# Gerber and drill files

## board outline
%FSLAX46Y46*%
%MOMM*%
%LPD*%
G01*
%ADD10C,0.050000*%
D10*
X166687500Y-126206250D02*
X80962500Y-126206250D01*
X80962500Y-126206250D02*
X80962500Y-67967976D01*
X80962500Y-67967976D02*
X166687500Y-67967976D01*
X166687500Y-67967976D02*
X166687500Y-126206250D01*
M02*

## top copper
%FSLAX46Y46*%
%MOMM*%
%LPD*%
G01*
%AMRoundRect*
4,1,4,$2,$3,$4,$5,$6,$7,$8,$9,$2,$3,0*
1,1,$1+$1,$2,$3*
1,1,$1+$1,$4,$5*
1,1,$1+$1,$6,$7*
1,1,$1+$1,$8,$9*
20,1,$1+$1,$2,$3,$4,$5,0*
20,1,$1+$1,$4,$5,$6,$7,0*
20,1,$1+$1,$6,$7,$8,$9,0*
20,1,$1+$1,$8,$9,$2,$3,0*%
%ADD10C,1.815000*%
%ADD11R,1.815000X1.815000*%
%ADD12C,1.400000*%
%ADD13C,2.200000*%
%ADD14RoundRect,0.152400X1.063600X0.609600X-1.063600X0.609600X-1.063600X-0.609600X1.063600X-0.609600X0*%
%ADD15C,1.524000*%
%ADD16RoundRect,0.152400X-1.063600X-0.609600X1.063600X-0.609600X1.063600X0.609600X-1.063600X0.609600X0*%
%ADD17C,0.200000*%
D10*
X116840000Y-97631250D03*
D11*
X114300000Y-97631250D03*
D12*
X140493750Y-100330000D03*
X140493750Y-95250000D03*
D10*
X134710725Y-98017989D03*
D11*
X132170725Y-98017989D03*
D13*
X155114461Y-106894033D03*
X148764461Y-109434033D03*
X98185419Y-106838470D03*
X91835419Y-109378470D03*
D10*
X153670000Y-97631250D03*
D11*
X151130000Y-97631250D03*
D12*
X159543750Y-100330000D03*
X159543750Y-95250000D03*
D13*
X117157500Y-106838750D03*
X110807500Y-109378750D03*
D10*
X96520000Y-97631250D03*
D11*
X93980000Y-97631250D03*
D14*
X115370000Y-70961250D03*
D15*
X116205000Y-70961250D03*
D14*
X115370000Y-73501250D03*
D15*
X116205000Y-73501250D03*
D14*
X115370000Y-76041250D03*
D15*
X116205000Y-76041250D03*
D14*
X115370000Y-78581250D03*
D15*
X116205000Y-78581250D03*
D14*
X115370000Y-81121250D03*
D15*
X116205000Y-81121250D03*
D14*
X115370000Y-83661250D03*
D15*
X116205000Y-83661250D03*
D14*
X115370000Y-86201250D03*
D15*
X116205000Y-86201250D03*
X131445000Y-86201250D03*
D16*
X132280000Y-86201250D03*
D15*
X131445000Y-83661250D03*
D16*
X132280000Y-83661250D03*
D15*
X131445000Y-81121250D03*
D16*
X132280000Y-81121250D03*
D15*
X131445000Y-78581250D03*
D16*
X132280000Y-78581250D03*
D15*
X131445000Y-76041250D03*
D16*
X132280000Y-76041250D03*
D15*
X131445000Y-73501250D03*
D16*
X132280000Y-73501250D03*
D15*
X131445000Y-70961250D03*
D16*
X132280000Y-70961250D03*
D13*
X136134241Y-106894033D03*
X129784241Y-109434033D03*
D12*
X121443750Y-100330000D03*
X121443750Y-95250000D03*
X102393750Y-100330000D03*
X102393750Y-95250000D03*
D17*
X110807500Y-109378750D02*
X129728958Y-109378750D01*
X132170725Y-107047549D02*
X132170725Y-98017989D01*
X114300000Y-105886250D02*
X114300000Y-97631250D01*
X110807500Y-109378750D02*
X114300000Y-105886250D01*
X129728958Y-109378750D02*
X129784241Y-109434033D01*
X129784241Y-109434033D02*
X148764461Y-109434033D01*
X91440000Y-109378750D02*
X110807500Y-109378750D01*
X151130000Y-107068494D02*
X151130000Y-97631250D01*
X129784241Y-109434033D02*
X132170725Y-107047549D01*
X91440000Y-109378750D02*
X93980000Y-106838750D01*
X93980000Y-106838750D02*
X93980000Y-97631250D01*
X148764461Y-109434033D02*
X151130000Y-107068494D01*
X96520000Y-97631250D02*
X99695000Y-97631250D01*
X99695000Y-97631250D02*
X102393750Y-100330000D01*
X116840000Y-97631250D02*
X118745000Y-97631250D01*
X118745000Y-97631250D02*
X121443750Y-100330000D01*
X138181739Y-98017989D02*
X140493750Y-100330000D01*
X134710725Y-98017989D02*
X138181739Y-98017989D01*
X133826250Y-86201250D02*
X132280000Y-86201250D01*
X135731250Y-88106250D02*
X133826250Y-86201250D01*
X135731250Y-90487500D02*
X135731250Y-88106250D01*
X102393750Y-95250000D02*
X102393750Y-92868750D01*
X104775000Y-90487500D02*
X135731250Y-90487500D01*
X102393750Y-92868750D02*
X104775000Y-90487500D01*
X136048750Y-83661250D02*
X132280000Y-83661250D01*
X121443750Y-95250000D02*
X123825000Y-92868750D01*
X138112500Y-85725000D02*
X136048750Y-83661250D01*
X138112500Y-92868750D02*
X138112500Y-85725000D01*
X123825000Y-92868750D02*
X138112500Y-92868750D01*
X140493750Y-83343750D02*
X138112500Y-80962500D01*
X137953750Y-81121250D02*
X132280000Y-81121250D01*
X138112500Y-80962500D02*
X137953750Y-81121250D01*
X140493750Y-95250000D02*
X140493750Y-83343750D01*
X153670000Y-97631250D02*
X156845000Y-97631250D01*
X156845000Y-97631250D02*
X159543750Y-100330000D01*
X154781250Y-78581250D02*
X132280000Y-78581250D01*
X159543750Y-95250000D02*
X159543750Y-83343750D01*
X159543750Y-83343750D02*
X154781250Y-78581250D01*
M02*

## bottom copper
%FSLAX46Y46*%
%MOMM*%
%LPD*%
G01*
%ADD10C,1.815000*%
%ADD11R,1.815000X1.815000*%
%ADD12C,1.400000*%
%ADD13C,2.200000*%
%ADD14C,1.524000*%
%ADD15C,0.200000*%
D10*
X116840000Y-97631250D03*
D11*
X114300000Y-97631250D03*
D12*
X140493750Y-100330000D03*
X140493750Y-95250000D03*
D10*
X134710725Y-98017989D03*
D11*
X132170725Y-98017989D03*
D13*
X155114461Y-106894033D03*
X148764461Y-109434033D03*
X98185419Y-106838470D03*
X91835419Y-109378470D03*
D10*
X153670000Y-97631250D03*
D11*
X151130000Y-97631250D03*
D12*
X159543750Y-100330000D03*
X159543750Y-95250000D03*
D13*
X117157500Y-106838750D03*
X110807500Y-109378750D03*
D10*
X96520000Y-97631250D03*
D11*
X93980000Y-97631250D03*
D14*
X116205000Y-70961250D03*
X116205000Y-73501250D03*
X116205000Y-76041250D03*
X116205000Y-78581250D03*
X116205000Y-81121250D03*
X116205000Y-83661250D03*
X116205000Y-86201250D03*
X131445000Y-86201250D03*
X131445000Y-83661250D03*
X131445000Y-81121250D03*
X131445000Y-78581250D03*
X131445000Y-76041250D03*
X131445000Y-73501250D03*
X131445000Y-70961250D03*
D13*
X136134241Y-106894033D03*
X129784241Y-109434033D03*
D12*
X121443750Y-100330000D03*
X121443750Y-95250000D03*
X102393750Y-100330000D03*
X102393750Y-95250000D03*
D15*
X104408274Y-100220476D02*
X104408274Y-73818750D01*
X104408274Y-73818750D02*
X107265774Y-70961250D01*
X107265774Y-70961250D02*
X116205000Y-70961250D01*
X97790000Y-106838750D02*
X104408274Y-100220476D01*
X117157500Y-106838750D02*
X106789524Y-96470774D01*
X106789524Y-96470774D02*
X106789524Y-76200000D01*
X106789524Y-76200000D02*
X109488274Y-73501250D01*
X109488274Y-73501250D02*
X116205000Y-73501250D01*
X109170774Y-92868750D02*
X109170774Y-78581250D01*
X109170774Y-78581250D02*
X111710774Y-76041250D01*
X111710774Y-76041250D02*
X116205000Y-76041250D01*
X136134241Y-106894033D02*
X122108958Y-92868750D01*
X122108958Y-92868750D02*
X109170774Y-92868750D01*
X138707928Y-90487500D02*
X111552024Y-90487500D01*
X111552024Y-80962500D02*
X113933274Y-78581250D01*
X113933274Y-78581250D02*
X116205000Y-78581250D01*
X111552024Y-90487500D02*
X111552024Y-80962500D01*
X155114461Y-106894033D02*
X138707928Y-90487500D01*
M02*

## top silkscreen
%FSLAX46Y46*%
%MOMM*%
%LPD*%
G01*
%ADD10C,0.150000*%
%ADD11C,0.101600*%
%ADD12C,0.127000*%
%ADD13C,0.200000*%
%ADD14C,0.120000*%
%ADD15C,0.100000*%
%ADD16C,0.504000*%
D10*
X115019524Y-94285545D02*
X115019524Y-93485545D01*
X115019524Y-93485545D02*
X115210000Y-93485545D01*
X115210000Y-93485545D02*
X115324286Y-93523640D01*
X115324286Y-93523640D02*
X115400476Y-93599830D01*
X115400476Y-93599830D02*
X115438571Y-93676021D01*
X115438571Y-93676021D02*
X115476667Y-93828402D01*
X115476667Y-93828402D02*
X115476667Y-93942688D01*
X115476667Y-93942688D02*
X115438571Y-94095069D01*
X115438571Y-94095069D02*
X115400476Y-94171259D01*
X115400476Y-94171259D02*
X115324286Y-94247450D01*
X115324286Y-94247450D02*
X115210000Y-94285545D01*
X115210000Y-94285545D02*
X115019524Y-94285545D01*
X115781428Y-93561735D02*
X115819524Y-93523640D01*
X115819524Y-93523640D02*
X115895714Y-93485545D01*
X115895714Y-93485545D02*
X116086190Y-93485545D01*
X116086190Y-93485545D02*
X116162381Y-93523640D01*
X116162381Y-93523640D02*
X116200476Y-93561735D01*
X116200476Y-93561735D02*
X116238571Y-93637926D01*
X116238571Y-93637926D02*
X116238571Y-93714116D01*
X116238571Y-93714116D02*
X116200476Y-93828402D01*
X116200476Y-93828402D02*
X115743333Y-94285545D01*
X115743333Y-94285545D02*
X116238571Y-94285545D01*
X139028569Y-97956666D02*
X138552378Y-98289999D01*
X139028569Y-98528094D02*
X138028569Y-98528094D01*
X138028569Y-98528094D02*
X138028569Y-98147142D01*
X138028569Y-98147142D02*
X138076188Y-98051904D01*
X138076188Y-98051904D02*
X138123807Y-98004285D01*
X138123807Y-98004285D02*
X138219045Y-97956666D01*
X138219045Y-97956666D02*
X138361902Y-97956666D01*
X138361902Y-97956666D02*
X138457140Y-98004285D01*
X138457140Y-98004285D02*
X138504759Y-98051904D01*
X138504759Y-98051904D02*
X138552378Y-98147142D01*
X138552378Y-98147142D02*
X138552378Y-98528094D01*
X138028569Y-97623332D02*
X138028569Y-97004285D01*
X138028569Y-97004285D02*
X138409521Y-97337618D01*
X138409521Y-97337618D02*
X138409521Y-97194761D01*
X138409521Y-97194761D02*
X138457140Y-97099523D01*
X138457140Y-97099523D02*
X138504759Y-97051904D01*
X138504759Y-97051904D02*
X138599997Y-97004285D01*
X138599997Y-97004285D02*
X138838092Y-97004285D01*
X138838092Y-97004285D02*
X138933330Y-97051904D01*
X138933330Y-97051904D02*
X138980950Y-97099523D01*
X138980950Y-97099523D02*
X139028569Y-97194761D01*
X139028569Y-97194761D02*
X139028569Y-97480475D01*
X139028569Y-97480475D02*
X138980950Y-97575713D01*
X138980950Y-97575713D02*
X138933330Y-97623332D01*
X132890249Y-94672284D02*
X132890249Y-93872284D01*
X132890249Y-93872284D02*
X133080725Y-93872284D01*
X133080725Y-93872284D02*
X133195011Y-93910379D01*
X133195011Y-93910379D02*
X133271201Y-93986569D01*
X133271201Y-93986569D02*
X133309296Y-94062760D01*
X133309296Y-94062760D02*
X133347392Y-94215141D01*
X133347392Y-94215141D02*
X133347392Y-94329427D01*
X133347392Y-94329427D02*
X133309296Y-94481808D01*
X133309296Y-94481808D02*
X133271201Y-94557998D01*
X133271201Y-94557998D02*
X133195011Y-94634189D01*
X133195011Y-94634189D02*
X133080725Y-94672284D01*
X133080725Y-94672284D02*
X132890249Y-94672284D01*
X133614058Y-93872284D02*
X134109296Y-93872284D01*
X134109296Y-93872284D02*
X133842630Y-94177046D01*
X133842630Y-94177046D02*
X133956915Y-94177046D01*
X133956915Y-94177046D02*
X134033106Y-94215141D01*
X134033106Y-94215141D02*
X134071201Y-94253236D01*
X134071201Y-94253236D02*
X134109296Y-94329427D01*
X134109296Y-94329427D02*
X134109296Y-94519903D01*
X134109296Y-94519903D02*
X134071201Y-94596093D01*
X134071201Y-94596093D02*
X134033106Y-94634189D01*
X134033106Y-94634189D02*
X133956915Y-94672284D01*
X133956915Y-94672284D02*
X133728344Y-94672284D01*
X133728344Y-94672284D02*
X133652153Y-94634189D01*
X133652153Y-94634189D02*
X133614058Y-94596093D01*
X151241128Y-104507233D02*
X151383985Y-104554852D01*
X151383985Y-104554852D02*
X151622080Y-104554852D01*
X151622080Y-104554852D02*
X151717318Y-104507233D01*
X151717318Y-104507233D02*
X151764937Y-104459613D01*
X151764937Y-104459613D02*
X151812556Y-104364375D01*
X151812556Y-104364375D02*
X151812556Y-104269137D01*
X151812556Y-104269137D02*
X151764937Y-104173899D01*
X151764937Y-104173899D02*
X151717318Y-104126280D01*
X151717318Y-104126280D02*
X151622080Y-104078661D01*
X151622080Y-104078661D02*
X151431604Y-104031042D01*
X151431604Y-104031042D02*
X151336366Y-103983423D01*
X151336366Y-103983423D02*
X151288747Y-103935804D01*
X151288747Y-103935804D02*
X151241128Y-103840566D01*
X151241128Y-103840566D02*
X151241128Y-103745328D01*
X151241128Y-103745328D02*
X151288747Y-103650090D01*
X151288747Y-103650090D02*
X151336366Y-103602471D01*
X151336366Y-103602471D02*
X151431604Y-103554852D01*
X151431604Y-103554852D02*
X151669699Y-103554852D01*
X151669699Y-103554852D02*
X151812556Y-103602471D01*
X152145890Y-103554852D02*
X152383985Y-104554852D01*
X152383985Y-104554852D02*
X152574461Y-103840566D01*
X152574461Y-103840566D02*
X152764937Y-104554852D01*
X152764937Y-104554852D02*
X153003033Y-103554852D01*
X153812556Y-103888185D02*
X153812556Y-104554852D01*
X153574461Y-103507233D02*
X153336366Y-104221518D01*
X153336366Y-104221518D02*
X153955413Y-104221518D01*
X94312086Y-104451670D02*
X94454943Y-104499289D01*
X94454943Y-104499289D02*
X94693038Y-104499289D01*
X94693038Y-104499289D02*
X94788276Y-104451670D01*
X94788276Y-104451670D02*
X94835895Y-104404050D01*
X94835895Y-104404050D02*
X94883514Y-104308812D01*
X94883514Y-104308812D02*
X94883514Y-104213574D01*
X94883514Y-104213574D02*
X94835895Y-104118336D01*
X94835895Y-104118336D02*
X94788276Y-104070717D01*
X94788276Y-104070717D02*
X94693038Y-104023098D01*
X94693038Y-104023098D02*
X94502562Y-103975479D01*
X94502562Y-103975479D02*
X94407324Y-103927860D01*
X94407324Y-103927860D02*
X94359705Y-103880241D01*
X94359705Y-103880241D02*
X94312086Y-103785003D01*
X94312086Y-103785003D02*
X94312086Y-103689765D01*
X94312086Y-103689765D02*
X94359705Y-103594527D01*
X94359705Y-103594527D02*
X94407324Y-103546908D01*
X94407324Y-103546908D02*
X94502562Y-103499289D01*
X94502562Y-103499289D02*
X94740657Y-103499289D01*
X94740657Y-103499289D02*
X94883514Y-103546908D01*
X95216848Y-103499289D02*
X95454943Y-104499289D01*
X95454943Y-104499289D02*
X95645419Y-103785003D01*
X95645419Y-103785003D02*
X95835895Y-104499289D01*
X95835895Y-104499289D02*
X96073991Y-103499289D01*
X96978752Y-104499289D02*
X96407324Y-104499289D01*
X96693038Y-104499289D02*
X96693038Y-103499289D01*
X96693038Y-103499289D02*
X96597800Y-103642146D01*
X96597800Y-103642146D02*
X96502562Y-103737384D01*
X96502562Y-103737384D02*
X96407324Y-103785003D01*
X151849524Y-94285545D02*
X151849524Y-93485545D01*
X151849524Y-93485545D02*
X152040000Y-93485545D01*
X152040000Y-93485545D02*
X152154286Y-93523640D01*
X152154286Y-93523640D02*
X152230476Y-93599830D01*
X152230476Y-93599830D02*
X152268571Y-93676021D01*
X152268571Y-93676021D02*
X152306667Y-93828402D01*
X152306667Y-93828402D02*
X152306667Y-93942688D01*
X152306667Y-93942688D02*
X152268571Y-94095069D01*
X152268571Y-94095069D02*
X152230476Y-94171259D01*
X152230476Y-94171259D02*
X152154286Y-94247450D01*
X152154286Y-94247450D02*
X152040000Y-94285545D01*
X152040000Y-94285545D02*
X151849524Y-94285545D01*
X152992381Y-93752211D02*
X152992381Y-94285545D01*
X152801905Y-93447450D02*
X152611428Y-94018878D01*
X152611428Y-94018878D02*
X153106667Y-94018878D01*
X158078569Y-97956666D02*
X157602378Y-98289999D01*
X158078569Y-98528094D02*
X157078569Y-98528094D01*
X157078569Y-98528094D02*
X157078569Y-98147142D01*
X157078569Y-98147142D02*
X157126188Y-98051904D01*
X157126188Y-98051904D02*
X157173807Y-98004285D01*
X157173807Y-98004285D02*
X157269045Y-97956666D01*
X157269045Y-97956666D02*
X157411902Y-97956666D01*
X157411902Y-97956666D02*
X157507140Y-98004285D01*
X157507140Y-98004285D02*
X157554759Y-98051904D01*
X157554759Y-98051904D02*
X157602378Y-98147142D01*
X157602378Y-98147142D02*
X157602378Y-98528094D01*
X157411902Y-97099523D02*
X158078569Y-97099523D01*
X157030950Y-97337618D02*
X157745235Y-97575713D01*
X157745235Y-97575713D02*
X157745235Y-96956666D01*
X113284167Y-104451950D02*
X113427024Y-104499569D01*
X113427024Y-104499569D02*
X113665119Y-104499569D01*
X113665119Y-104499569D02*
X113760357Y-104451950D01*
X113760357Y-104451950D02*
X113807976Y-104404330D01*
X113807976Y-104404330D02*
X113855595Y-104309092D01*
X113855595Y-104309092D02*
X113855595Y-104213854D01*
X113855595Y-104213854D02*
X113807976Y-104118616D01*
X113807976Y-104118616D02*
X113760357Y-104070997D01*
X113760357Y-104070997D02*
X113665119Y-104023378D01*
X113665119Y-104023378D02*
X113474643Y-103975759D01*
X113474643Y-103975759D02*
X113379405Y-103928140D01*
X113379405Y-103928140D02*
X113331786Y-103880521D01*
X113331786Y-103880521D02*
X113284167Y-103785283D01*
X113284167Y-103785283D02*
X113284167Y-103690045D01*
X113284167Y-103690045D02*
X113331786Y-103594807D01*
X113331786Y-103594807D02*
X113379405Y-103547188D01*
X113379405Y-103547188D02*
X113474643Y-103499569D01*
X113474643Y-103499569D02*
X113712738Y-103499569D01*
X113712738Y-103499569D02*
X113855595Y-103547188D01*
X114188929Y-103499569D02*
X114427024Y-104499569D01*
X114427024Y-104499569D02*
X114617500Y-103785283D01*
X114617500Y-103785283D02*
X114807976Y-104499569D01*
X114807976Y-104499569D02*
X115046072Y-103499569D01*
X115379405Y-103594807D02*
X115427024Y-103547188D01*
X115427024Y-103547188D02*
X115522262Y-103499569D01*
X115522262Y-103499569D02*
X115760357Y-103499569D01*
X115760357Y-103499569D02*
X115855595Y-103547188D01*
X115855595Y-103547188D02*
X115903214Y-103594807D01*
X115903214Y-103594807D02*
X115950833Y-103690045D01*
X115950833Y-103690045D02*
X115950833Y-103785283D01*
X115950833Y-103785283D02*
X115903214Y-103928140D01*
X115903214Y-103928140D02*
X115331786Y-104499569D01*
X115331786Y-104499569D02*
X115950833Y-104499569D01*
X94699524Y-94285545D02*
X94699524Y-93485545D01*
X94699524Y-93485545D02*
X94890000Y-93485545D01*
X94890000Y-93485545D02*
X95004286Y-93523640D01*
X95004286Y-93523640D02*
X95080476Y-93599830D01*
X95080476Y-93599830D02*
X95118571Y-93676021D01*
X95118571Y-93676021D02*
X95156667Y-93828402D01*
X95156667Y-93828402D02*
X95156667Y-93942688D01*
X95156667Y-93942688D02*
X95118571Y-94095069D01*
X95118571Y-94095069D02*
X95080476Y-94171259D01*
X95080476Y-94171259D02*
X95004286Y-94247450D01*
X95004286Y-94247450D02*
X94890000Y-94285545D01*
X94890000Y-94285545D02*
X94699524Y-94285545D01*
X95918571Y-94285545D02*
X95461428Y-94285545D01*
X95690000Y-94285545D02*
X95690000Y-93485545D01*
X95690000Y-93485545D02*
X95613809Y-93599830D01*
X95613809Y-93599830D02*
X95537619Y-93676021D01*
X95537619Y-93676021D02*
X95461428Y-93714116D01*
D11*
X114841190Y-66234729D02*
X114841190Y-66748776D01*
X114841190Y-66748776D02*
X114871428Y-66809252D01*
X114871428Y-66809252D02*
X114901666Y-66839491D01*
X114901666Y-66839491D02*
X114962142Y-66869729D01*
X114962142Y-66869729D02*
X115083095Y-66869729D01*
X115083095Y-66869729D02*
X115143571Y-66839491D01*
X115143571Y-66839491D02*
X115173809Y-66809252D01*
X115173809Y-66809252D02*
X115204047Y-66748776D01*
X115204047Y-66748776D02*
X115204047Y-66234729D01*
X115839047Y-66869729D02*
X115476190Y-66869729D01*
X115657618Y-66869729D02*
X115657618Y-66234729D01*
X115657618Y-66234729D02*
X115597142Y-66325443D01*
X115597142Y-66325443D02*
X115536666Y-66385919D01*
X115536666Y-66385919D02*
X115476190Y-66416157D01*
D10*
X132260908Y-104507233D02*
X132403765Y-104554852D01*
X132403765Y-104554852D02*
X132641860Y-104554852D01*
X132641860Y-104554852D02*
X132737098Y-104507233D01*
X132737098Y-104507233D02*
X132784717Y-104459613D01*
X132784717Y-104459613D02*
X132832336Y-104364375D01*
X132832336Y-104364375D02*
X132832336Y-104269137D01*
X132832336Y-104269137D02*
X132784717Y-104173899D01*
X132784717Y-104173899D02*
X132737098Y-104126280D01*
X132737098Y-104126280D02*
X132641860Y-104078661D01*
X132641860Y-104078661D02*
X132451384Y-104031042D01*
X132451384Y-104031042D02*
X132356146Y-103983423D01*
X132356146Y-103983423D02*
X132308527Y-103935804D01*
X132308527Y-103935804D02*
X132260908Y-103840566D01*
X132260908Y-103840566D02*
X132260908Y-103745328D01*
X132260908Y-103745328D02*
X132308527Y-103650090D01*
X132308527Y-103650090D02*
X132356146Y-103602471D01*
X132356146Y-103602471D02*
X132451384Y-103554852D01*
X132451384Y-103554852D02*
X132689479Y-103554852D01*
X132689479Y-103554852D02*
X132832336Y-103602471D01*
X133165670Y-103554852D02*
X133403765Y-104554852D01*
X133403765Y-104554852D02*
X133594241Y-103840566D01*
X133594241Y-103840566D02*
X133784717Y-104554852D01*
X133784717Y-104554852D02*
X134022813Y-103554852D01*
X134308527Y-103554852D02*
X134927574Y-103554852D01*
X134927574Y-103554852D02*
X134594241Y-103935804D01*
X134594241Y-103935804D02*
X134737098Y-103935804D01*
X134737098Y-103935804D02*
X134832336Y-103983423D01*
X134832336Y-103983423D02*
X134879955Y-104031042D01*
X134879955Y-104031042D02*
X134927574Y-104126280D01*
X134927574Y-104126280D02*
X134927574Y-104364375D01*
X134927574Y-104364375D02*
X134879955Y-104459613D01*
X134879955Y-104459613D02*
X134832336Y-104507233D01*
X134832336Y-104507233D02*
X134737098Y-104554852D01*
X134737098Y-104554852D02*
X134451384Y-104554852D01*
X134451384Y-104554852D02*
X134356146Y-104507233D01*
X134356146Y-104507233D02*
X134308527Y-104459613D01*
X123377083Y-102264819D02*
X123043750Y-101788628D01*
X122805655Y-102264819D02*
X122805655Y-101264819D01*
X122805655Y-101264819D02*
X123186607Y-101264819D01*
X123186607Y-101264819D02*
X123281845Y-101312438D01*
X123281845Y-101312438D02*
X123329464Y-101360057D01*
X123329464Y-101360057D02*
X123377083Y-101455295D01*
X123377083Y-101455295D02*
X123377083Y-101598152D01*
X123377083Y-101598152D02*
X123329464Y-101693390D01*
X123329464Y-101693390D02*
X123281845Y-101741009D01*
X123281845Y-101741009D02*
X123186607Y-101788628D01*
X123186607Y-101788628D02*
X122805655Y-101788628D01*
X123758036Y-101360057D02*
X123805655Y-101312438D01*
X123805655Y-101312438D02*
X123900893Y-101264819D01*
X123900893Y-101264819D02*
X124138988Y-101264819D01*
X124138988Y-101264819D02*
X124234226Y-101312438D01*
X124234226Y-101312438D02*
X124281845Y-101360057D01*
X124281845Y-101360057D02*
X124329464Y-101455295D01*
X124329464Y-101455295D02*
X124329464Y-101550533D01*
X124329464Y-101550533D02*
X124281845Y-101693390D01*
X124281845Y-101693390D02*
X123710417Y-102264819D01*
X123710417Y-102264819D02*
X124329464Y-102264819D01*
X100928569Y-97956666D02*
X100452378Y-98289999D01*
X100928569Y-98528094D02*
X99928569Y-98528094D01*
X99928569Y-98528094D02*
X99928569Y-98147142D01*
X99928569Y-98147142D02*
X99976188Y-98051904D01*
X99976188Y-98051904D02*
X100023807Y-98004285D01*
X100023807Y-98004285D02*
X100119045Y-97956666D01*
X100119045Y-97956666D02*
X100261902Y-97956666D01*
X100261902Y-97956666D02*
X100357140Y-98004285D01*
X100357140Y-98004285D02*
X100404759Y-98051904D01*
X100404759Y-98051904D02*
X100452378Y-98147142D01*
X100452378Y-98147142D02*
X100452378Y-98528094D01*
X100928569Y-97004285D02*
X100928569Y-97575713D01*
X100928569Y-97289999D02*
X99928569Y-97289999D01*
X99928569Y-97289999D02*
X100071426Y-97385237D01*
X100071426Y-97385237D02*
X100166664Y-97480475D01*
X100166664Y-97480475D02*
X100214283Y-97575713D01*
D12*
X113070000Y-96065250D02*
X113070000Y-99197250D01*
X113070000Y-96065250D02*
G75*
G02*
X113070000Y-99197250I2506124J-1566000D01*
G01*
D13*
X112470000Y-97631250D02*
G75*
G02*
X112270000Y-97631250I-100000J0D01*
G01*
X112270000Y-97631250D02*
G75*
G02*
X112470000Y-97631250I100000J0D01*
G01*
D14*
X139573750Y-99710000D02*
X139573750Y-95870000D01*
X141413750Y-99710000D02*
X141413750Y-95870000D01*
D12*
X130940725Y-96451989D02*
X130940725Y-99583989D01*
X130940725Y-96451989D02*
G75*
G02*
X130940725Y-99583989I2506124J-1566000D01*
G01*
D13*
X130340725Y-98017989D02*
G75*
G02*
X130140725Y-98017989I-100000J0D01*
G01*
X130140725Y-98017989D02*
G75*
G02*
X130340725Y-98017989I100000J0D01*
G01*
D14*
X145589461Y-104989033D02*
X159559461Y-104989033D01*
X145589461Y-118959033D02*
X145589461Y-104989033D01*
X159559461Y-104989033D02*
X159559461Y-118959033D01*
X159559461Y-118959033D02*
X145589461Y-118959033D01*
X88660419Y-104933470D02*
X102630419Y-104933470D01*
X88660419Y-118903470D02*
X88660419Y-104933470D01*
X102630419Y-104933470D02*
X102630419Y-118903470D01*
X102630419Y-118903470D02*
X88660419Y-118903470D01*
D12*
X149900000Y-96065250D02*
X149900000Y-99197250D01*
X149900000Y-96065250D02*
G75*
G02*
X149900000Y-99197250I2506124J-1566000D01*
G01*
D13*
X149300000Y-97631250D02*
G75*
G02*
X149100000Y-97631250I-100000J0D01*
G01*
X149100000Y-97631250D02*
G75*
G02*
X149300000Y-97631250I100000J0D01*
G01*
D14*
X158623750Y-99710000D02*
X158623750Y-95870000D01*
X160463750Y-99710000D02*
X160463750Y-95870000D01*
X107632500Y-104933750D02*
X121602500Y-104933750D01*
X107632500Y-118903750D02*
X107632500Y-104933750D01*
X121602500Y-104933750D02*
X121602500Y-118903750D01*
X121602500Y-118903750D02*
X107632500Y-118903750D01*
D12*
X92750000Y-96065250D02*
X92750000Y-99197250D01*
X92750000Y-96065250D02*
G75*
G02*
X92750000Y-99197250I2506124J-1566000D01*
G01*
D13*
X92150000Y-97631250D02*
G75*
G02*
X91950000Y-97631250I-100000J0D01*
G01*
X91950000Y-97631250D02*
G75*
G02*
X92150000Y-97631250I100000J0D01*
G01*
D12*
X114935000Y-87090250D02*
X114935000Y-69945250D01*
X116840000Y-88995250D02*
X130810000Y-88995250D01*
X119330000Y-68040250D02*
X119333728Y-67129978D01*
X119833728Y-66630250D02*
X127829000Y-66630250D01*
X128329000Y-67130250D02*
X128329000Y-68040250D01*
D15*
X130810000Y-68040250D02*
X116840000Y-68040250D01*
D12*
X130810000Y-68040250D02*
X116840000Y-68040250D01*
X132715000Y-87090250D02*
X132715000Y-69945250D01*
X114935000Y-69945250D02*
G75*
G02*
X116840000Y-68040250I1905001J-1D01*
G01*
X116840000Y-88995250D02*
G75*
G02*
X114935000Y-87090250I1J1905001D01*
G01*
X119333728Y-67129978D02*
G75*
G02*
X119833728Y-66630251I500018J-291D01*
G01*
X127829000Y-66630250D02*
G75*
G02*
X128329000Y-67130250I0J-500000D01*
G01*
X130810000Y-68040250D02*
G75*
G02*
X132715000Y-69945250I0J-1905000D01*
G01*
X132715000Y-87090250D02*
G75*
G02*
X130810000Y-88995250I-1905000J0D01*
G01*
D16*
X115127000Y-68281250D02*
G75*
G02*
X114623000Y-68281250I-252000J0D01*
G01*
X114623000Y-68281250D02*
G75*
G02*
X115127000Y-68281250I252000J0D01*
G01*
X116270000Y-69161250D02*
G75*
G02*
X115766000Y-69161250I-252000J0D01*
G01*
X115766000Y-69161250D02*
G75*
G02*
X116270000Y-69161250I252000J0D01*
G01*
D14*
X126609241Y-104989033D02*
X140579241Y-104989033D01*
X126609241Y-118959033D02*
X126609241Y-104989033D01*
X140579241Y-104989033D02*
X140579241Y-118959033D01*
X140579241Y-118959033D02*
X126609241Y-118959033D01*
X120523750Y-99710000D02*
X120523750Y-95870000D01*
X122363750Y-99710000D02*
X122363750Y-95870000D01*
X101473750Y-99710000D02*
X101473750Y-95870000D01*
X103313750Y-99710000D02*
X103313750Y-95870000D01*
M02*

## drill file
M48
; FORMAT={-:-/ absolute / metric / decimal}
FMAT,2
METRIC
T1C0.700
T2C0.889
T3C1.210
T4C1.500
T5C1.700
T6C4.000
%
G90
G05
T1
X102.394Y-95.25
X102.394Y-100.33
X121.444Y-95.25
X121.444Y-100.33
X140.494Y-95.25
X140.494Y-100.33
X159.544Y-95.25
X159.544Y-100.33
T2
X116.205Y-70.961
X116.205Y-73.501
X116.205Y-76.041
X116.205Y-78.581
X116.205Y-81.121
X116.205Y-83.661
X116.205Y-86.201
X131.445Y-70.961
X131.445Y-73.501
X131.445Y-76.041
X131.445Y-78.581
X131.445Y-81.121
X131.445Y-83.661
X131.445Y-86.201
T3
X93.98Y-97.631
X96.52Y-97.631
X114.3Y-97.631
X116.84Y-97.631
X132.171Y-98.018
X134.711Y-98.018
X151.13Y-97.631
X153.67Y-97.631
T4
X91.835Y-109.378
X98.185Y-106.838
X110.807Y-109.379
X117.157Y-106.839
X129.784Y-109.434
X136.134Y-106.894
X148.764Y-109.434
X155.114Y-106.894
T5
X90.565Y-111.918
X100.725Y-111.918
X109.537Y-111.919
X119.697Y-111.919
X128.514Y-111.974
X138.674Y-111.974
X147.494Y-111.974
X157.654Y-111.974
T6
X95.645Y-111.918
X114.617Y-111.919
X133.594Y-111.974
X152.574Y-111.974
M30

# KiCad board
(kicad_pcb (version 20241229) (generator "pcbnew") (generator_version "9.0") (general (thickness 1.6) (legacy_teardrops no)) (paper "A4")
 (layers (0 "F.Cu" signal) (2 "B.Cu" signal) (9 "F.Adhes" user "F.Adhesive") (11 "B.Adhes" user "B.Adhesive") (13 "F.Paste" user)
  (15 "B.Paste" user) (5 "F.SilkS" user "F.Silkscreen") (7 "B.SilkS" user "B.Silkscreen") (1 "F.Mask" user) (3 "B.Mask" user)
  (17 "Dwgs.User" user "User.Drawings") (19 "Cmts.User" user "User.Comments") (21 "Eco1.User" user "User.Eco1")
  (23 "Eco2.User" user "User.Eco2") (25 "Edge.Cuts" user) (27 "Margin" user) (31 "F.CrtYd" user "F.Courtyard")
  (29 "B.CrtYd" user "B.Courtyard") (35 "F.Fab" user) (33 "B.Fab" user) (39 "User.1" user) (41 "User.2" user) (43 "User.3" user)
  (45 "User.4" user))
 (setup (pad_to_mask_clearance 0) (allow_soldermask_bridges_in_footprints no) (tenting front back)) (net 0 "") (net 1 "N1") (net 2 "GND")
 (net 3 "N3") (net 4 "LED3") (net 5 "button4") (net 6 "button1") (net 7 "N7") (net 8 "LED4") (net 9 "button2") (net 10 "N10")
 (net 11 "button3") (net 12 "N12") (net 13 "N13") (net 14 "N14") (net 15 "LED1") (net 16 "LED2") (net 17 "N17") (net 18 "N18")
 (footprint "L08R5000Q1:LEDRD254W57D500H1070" (layer "F.Cu") (at 115.57 97.63125)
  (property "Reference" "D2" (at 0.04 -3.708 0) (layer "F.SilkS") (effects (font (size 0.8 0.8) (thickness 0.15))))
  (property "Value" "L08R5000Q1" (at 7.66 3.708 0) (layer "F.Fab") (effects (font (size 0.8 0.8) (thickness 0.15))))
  (fp_line (start -2.5 -1.566) (end -2.5 1.566) (stroke (width 0.127) (type solid)) (layer "F.SilkS"))
  (fp_arc (start -2.5 -1.566) (mid 2.961291 0) (end -2.5 1.566) (stroke (width 0.127) (type solid)) (layer "F.SilkS"))
  (fp_circle (center -3.2 0) (end -3.1 0) (stroke (width 0.2) (type solid)) (fill no) (layer "F.SilkS"))
  (pad "A" thru_hole circle (at 1.27 0) (size 1.815 1.815) (drill 1.21) (layers "*.Cu" "*.Mask") (remove_unused_layers no) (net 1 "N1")
   (solder_mask_margin 0.102))
  (pad "C" thru_hole rect (at -1.27 0) (size 1.815 1.815) (drill 1.21) (layers "*.Cu" "*.Mask") (remove_unused_layers no) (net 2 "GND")
   (solder_mask_margin 0.102)))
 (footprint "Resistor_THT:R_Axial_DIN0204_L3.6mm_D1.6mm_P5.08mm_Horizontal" (layer "F.Cu") (at 140.49375 100.33 90)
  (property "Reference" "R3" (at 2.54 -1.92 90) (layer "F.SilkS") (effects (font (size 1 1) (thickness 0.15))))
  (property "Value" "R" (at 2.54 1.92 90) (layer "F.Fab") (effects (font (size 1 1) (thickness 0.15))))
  (fp_line (start 0.62 -0.92) (end 4.46 -0.92) (stroke (width 0.12) (type solid)) (layer "F.SilkS"))
  (fp_line (start 0.62 0.92) (end 4.46 0.92) (stroke (width 0.12) (type solid)) (layer "F.SilkS"))
  (pad "1" thru_hole circle (at 0 0 90) (size 1.4 1.4) (drill 0.7) (layers "*.Cu" "*.Mask") (remove_unused_layers no) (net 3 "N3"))
  (pad "2" thru_hole circle (at 5.08 0 90) (size 1.4 1.4) (drill 0.7) (layers "*.Cu" "*.Mask") (remove_unused_layers no) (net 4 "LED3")))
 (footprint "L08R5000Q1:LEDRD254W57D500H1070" (layer "F.Cu") (at 133.440725 98.017989)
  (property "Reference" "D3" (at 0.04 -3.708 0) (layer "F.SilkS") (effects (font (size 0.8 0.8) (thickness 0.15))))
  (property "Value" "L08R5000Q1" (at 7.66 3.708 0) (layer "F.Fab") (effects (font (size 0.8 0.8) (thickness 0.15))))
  (fp_line (start -2.5 -1.566) (end -2.5 1.566) (stroke (width 0.127) (type solid)) (layer "F.SilkS"))
  (fp_arc (start -2.5 -1.566) (mid 2.961291 0) (end -2.5 1.566) (stroke (width 0.127) (type solid)) (layer "F.SilkS"))
  (fp_circle (center -3.2 0) (end -3.1 0) (stroke (width 0.2) (type solid)) (fill no) (layer "F.SilkS"))
  (pad "A" thru_hole circle (at 1.27 0) (size 1.815 1.815) (drill 1.21) (layers "*.Cu" "*.Mask") (remove_unused_layers no) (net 3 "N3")
   (solder_mask_margin 0.102))
  (pad "C" thru_hole rect (at -1.27 0) (size 1.815 1.815) (drill 1.21) (layers "*.Cu" "*.Mask") (remove_unused_layers no) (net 2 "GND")
   (solder_mask_margin 0.102)))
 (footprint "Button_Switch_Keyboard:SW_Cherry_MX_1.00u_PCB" (layer "F.Cu") (at 155.114461 106.894033)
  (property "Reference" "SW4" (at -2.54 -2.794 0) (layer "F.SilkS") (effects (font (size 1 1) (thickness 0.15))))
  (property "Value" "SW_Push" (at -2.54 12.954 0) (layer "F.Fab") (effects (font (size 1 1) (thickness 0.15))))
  (fp_line (start -9.525 -1.905) (end 4.445 -1.905) (stroke (width 0.12) (type solid)) (layer "F.SilkS"))
  (fp_line (start -9.525 12.065) (end -9.525 -1.905) (stroke (width 0.12) (type solid)) (layer "F.SilkS"))
  (fp_line (start 4.445 -1.905) (end 4.445 12.065) (stroke (width 0.12) (type solid)) (layer "F.SilkS"))
  (fp_line (start 4.445 12.065) (end -9.525 12.065) (stroke (width 0.12) (type solid)) (layer "F.SilkS"))
  (pad "" np_thru_hole circle (at -7.62 5.08) (size 1.7 1.7) (drill 1.7) (layers "*.Cu" "*.Mask"))
  (pad "" np_thru_hole circle (at -2.54 5.08) (size 4 4) (drill 4) (layers "*.Cu" "*.Mask"))
  (pad "" np_thru_hole circle (at 2.54 5.08) (size 1.7 1.7) (drill 1.7) (layers "*.Cu" "*.Mask"))
  (pad "1" thru_hole circle (at 0 0) (size 2.2 2.2) (drill 1.5) (layers "*.Cu" "*.Mask") (remove_unused_layers no) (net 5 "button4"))
  (pad "2" thru_hole circle (at -6.35 2.54) (size 2.2 2.2) (drill 1.5) (layers "*.Cu" "*.Mask") (remove_unused_layers no) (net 2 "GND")))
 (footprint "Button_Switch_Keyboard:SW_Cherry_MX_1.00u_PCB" (layer "F.Cu") (at 98.185419 106.83847)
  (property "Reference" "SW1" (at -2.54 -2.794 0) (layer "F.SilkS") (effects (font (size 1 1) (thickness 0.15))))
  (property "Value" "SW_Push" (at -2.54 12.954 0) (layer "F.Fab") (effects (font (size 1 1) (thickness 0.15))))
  (fp_line (start -9.525 -1.905) (end 4.445 -1.905) (stroke (width 0.12) (type solid)) (layer "F.SilkS"))
  (fp_line (start -9.525 12.065) (end -9.525 -1.905) (stroke (width 0.12) (type solid)) (layer "F.SilkS"))
  (fp_line (start 4.445 -1.905) (end 4.445 12.065) (stroke (width 0.12) (type solid)) (layer "F.SilkS"))
  (fp_line (start 4.445 12.065) (end -9.525 12.065) (stroke (width 0.12) (type solid)) (layer "F.SilkS"))
  (pad "" np_thru_hole circle (at -7.62 5.08) (size 1.7 1.7) (drill 1.7) (layers "*.Cu" "*.Mask"))
  (pad "" np_thru_hole circle (at -2.54 5.08) (size 4 4) (drill 4) (layers "*.Cu" "*.Mask"))
  (pad "" np_thru_hole circle (at 2.54 5.08) (size 1.7 1.7) (drill 1.7) (layers "*.Cu" "*.Mask"))
  (pad "1" thru_hole circle (at 0 0) (size 2.2 2.2) (drill 1.5) (layers "*.Cu" "*.Mask") (remove_unused_layers no) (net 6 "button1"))
  (pad "2" thru_hole circle (at -6.35 2.54) (size 2.2 2.2) (drill 1.5) (layers "*.Cu" "*.Mask") (remove_unused_layers no) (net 2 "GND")))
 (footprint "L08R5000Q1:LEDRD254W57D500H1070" (layer "F.Cu") (at 152.4 97.63125)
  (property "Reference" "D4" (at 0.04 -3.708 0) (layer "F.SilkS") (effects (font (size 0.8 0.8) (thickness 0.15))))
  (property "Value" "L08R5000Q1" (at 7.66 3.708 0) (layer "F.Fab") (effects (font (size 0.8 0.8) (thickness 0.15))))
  (fp_line (start -2.5 -1.566) (end -2.5 1.566) (stroke (width 0.127) (type solid)) (layer "F.SilkS"))
  (fp_arc (start -2.5 -1.566) (mid 2.961291 0) (end -2.5 1.566) (stroke (width 0.127) (type solid)) (layer "F.SilkS"))
  (fp_circle (center -3.2 0) (end -3.1 0) (stroke (width 0.2) (type solid)) (fill no) (layer "F.SilkS"))
  (pad "A" thru_hole circle (at 1.27 0) (size 1.815 1.815) (drill 1.21) (layers "*.Cu" "*.Mask") (remove_unused_layers no) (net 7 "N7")
   (solder_mask_margin 0.102))
  (pad "C" thru_hole rect (at -1.27 0) (size 1.815 1.815) (drill 1.21) (layers "*.Cu" "*.Mask") (remove_unused_layers no) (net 2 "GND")
   (solder_mask_margin 0.102)))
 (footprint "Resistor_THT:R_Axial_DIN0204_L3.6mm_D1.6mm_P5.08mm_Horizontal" (layer "F.Cu") (at 159.54375 100.33 90)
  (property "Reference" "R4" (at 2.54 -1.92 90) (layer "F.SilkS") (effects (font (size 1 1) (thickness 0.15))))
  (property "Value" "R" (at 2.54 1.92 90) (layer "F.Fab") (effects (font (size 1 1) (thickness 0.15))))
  (fp_line (start 0.62 -0.92) (end 4.46 -0.92) (stroke (width 0.12) (type solid)) (layer "F.SilkS"))
  (fp_line (start 0.62 0.92) (end 4.46 0.92) (stroke (width 0.12) (type solid)) (layer "F.SilkS"))
  (pad "1" thru_hole circle (at 0 0 90) (size 1.4 1.4) (drill 0.7) (layers "*.Cu" "*.Mask") (remove_unused_layers no) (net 7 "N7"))
  (pad "2" thru_hole circle (at 5.08 0 90) (size 1.4 1.4) (drill 0.7) (layers "*.Cu" "*.Mask") (remove_unused_layers no) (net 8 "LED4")))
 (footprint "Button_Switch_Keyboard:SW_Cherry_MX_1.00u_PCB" (layer "F.Cu") (at 117.1575 106.83875)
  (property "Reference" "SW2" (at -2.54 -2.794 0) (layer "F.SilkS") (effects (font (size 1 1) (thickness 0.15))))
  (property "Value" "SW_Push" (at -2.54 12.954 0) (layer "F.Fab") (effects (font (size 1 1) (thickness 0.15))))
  (fp_line (start -9.525 -1.905) (end 4.445 -1.905) (stroke (width 0.12) (type solid)) (layer "F.SilkS"))
  (fp_line (start -9.525 12.065) (end -9.525 -1.905) (stroke (width 0.12) (type solid)) (layer "F.SilkS"))
  (fp_line (start 4.445 -1.905) (end 4.445 12.065) (stroke (width 0.12) (type solid)) (layer "F.SilkS"))
  (fp_line (start 4.445 12.065) (end -9.525 12.065) (stroke (width 0.12) (type solid)) (layer "F.SilkS"))
  (pad "" np_thru_hole circle (at -7.62 5.08) (size 1.7 1.7) (drill 1.7) (layers "*.Cu" "*.Mask"))
  (pad "" np_thru_hole circle (at -2.54 5.08) (size 4 4) (drill 4) (layers "*.Cu" "*.Mask"))
  (pad "" np_thru_hole circle (at 2.54 5.08) (size 1.7 1.7) (drill 1.7) (layers "*.Cu" "*.Mask"))
  (pad "1" thru_hole circle (at 0 0) (size 2.2 2.2) (drill 1.5) (layers "*.Cu" "*.Mask") (remove_unused_layers no) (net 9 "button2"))
  (pad "2" thru_hole circle (at -6.35 2.54) (size 2.2 2.2) (drill 1.5) (layers "*.Cu" "*.Mask") (remove_unused_layers no) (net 2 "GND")))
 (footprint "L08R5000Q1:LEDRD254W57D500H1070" (layer "F.Cu") (at 95.25 97.63125)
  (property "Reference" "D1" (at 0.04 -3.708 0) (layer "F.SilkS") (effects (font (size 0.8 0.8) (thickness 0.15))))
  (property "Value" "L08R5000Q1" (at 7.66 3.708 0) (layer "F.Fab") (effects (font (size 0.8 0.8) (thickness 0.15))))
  (fp_line (start -2.5 -1.566) (end -2.5 1.566) (stroke (width 0.127) (type solid)) (layer "F.SilkS"))
  (fp_arc (start -2.5 -1.566) (mid 2.961291 0) (end -2.5 1.566) (stroke (width 0.127) (type solid)) (layer "F.SilkS"))
  (fp_circle (center -3.2 0) (end -3.1 0) (stroke (width 0.2) (type solid)) (fill no) (layer "F.SilkS"))
  (pad "A" thru_hole circle (at 1.27 0) (size 1.815 1.815) (drill 1.21) (layers "*.Cu" "*.Mask") (remove_unused_layers no) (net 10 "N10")
   (solder_mask_margin 0.102))
  (pad "C" thru_hole rect (at -1.27 0) (size 1.815 1.815) (drill 1.21) (layers "*.Cu" "*.Mask") (remove_unused_layers no) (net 2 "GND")
   (solder_mask_margin 0.102)))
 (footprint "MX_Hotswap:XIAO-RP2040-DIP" (layer "F.Cu") (at 123.825 78.58125)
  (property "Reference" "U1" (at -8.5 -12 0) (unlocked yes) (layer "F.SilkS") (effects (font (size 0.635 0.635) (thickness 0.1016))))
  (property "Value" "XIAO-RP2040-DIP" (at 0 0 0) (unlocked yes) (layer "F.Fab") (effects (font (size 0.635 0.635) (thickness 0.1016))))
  (fp_line (start -8.89 8.509) (end -8.89 -8.636) (stroke (width 0.127) (type solid)) (layer "F.SilkS"))
  (fp_line (start -6.985 10.414) (end 6.985 10.414) (stroke (width 0.127) (type solid)) (layer "F.SilkS"))
  (fp_line (start -4.495 -10.541) (end -4.491272 -11.451272) (stroke (width 0.127) (type solid)) (layer "F.SilkS"))
  (fp_line (start -3.991272 -11.951) (end 4.004 -11.951) (stroke (width 0.127) (type solid)) (layer "F.SilkS"))
  (fp_line (start 4.504 -11.451) (end 4.504 -10.541) (stroke (width 0.127) (type solid)) (layer "F.SilkS"))
  (fp_line (start 6.985 -10.541) (end -6.985 -10.541) (stroke (width 0.1) (type solid)) (layer "F.SilkS"))
  (fp_line (start 6.985 -10.541) (end -6.985 -10.541) (stroke (width 0.127) (type solid)) (layer "F.SilkS"))
  (fp_line (start 8.89 8.509) (end 8.89 -8.636) (stroke (width 0.127) (type solid)) (layer "F.SilkS"))
  (fp_arc (start -8.89 -8.636) (mid -8.332038 -9.983038) (end -6.985 -10.541) (stroke (width 0.127) (type solid)) (layer "F.SilkS"))
  (fp_arc (start -6.985 10.414) (mid -8.332038 9.856038) (end -8.89 8.509) (stroke (width 0.127) (type solid)) (layer "F.SilkS"))
  (fp_arc (start -4.491272 -11.451272) (mid -4.344728 -11.80464) (end -3.991272 -11.951) (stroke (width 0.127) (type default))
   (layer "F.SilkS"))
  (fp_arc (start 4.004 -11.951) (mid 4.357553 -11.804553) (end 4.504 -11.451) (stroke (width 0.127) (type default)) (layer "F.SilkS"))
  (fp_arc (start 6.985 -10.541) (mid 8.332038 -9.983038) (end 8.89 -8.636) (stroke (width 0.127) (type solid)) (layer "F.SilkS"))
  (fp_arc (start 8.89 8.509) (mid 8.332038 9.856038) (end 6.985 10.414) (stroke (width 0.127) (type solid)) (layer "F.SilkS"))
  (fp_circle (center -8.95 -10.3) (end -8.95 -10.554) (stroke (width 0.5) (type solid)) (fill yes) (layer "F.SilkS"))
  (fp_circle (center -7.807 -9.42) (end -7.807 -9.674) (stroke (width 0.5) (type solid)) (fill yes) (layer "F.SilkS"))
  (pad "1" smd roundrect (at -8.455 -7.62 180) (size 2.432 1.524) (layers "F.Cu" "F.Mask") (roundrect_rratio 0.1) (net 6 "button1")
   (thermal_bridge_angle 45))
  (pad "1" thru_hole circle (at -7.62 -7.62 180) (size 1.524 1.524) (drill 0.889) (layers "*.Cu" "*.Mask") (remove_unused_layers no)
   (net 6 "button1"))
  (pad "2" smd roundrect (at -8.455 -5.08 180) (size 2.432 1.524) (layers "F.Cu" "F.Mask") (roundrect_rratio 0.1) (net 9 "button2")
   (thermal_bridge_angle 45))
  (pad "2" thru_hole circle (at -7.62 -5.08 180) (size 1.524 1.524) (drill 0.889) (layers "*.Cu" "*.Mask") (remove_unused_layers no)
   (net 9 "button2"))
  (pad "3" smd roundrect (at -8.455 -2.54 180) (size 2.432 1.524) (layers "F.Cu" "F.Mask") (roundrect_rratio 0.1) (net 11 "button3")
   (thermal_bridge_angle 45))
  (pad "3" thru_hole circle (at -7.62 -2.54 180) (size 1.524 1.524) (drill 0.889) (layers "*.Cu" "*.Mask") (remove_unused_layers no)
   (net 11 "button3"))
  (pad "4" smd roundrect (at -8.455 0 180) (size 2.432 1.524) (layers "F.Cu" "F.Mask") (roundrect_rratio 0.1) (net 5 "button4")
   (thermal_bridge_angle 45))
  (pad "4" thru_hole circle (at -7.62 0 180) (size 1.524 1.524) (drill 0.889) (layers "*.Cu" "*.Mask") (remove_unused_layers no)
   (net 5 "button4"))
  (pad "5" smd roundrect (at -8.455 2.54 180) (size 2.432 1.524) (layers "F.Cu" "F.Mask") (roundrect_rratio 0.1) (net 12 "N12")
   (thermal_bridge_angle 45))
  (pad "5" thru_hole circle (at -7.62 2.54 180) (size 1.524 1.524) (drill 0.889) (layers "*.Cu" "*.Mask") (remove_unused_layers no)
   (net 12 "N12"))
  (pad "6" smd roundrect (at -8.455 5.08 180) (size 2.432 1.524) (layers "F.Cu" "F.Mask") (roundrect_rratio 0.1) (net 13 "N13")
   (thermal_bridge_angle 45))
  (pad "6" thru_hole circle (at -7.62 5.08 180) (size 1.524 1.524) (drill 0.889) (layers "*.Cu" "*.Mask") (remove_unused_layers no)
   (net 13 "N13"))
  (pad "7" smd roundrect (at -8.455 7.62 180) (size 2.432 1.524) (layers "F.Cu" "F.Mask") (roundrect_rratio 0.1) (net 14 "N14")
   (thermal_bridge_angle 45))
  (pad "7" thru_hole circle (at -7.62 7.62 180) (size 1.524 1.524) (drill 0.889) (layers "*.Cu" "*.Mask") (remove_unused_layers no)
   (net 14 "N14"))
  (pad "8" thru_hole circle (at 7.62 7.62) (size 1.524 1.524) (drill 0.889) (layers "*.Cu" "*.Mask") (remove_unused_layers no)
   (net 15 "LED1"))
  (pad "8" smd roundrect (at 8.455 7.62) (size 2.432 1.524) (layers "F.Cu" "F.Mask") (roundrect_rratio 0.1) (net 15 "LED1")
   (thermal_bridge_angle 45))
  (pad "9" thru_hole circle (at 7.62 5.08) (size 1.524 1.524) (drill 0.889) (layers "*.Cu" "*.Mask") (remove_unused_layers no)
   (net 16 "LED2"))
  (pad "9" smd roundrect (at 8.455 5.08) (size 2.432 1.524) (layers "F.Cu" "F.Mask") (roundrect_rratio 0.1) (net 16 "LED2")
   (thermal_bridge_angle 45))
  (pad "10" thru_hole circle (at 7.62 2.54) (size 1.524 1.524) (drill 0.889) (layers "*.Cu" "*.Mask") (remove_unused_layers no)
   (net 4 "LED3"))
  (pad "10" smd roundrect (at 8.455 2.54) (size 2.432 1.524) (layers "F.Cu" "F.Mask") (roundrect_rratio 0.1) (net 4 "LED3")
   (thermal_bridge_angle 45))
  (pad "11" thru_hole circle (at 7.62 0) (size 1.524 1.524) (drill 0.889) (layers "*.Cu" "*.Mask") (remove_unused_layers no) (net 8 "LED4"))
  (pad "11" smd roundrect (at 8.455 0) (size 2.432 1.524) (layers "F.Cu" "F.Mask") (roundrect_rratio 0.1) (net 8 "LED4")
   (thermal_bridge_angle 45))
  (pad "12" thru_hole circle (at 7.62 -2.54) (size 1.524 1.524) (drill 0.889) (layers "*.Cu" "*.Mask") (remove_unused_layers no)
   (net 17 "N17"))
  (pad "12" smd roundrect (at 8.455 -2.54) (size 2.432 1.524) (layers "F.Cu" "F.Mask") (roundrect_rratio 0.1) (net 17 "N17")
   (thermal_bridge_angle 45))
  (pad "13" thru_hole circle (at 7.62 -5.08) (size 1.524 1.524) (drill 0.889) (layers "*.Cu" "*.Mask") (remove_unused_layers no)
   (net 2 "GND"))
  (pad "13" smd roundrect (at 8.455 -5.08) (size 2.432 1.524) (layers "F.Cu" "F.Mask") (roundrect_rratio 0.1) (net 2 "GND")
   (thermal_bridge_angle 45))
  (pad "14" thru_hole circle (at 7.62 -7.62) (size 1.524 1.524) (drill 0.889) (layers "*.Cu" "*.Mask") (remove_unused_layers no)
   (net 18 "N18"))
  (pad "14" smd roundrect (at 8.455 -7.62) (size 2.432 1.524) (layers "F.Cu" "F.Mask") (roundrect_rratio 0.1) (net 18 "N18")
   (thermal_bridge_angle 45)))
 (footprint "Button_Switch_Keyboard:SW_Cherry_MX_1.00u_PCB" (layer "F.Cu") (at 136.134241 106.894033)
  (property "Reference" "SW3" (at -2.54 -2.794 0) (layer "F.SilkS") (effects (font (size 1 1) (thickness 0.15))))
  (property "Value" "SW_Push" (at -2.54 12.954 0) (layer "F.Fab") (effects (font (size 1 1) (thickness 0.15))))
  (fp_line (start -9.525 -1.905) (end 4.445 -1.905) (stroke (width 0.12) (type solid)) (layer "F.SilkS"))
  (fp_line (start -9.525 12.065) (end -9.525 -1.905) (stroke (width 0.12) (type solid)) (layer "F.SilkS"))
  (fp_line (start 4.445 -1.905) (end 4.445 12.065) (stroke (width 0.12) (type solid)) (layer "F.SilkS"))
  (fp_line (start 4.445 12.065) (end -9.525 12.065) (stroke (width 0.12) (type solid)) (layer "F.SilkS"))
  (pad "" np_thru_hole circle (at -7.62 5.08) (size 1.7 1.7) (drill 1.7) (layers "*.Cu" "*.Mask"))
  (pad "" np_thru_hole circle (at -2.54 5.08) (size 4 4) (drill 4) (layers "*.Cu" "*.Mask"))
  (pad "" np_thru_hole circle (at 2.54 5.08) (size 1.7 1.7) (drill 1.7) (layers "*.Cu" "*.Mask"))
  (pad "1" thru_hole circle (at 0 0) (size 2.2 2.2) (drill 1.5) (layers "*.Cu" "*.Mask") (remove_unused_layers no) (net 11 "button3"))
  (pad "2" thru_hole circle (at -6.35 2.54) (size 2.2 2.2) (drill 1.5) (layers "*.Cu" "*.Mask") (remove_unused_layers no) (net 2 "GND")))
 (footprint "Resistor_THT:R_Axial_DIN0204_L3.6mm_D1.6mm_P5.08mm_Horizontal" (layer "F.Cu") (at 121.44375 100.33 90)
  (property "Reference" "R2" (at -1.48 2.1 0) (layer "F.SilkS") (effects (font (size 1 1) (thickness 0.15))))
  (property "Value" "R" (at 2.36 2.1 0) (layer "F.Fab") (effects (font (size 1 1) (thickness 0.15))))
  (fp_line (start 0.62 -0.92) (end 4.46 -0.92) (stroke (width 0.12) (type solid)) (layer "F.SilkS"))
  (fp_line (start 0.62 0.92) (end 4.46 0.92) (stroke (width 0.12) (type solid)) (layer "F.SilkS"))
  (pad "1" thru_hole circle (at 0 0 90) (size 1.4 1.4) (drill 0.7) (layers "*.Cu" "*.Mask") (remove_unused_layers no) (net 1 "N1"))
  (pad "2" thru_hole circle (at 5.08 0 90) (size 1.4 1.4) (drill 0.7) (layers "*.Cu" "*.Mask") (remove_unused_layers no) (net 16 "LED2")))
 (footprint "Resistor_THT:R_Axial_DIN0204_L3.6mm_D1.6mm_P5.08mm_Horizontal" (layer "F.Cu") (at 102.39375 100.33 90)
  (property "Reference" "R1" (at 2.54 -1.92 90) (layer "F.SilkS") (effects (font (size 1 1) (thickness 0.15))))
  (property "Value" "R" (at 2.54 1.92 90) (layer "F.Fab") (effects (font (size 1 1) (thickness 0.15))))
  (fp_line (start 0.62 -0.92) (end 4.46 -0.92) (stroke (width 0.12) (type solid)) (layer "F.SilkS"))
  (fp_line (start 0.62 0.92) (end 4.46 0.92) (stroke (width 0.12) (type solid)) (layer "F.SilkS"))
  (pad "1" thru_hole circle (at 0 0 90) (size 1.4 1.4) (drill 0.7) (layers "*.Cu" "*.Mask") (remove_unused_layers no) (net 10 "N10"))
  (pad "2" thru_hole circle (at 5.08 0 90) (size 1.4 1.4) (drill 0.7) (layers "*.Cu" "*.Mask") (remove_unused_layers no) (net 15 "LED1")))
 (gr_line (start 166.6875 126.20625) (end 80.9625 126.20625) (stroke (width 0.05) (type default)) (layer "Edge.Cuts"))
 (gr_line (start 80.9625 126.20625) (end 80.9625 67.967976) (stroke (width 0.05) (type default)) (layer "Edge.Cuts"))
 (gr_line (start 80.9625 67.967976) (end 166.6875 67.967976) (stroke (width 0.05) (type default)) (layer "Edge.Cuts"))
 (gr_line (start 166.6875 67.967976) (end 166.6875 126.20625) (stroke (width 0.05) (type default)) (layer "Edge.Cuts"))
 (segment (start 110.8075 109.37875) (end 129.728958 109.37875) (width 0.2) (layer "F.Cu") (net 2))
 (segment (start 132.170725 107.047549) (end 132.170725 98.017989) (width 0.2) (layer "F.Cu") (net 2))
 (segment (start 114.3 105.88625) (end 114.3 97.63125) (width 0.2) (layer "F.Cu") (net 2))
 (segment (start 110.8075 109.37875) (end 114.3 105.88625) (width 0.2) (layer "F.Cu") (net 2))
 (segment (start 129.728958 109.37875) (end 129.784241 109.434033) (width 0.2) (layer "F.Cu") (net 2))
 (segment (start 129.784241 109.434033) (end 148.764461 109.434033) (width 0.2) (layer "F.Cu") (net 2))
 (segment (start 91.44 109.37875) (end 110.8075 109.37875) (width 0.2) (layer "F.Cu") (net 2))
 (segment (start 151.13 107.068494) (end 151.13 97.63125) (width 0.2) (layer "F.Cu") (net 2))
 (segment (start 129.784241 109.434033) (end 132.170725 107.047549) (width 0.2) (layer "F.Cu") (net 2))
 (segment (start 91.44 109.37875) (end 93.98 106.83875) (width 0.2) (layer "F.Cu") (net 2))
 (segment (start 93.98 106.83875) (end 93.98 97.63125) (width 0.2) (layer "F.Cu") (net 2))
 (segment (start 148.764461 109.434033) (end 151.13 107.068494) (width 0.2) (layer "F.Cu") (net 2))
 (segment (start 96.52 97.63125) (end 99.695 97.63125) (width 0.2) (layer "F.Cu") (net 10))
 (segment (start 99.695 97.63125) (end 102.39375 100.33) (width 0.2) (layer "F.Cu") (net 10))
 (segment (start 116.84 97.63125) (end 118.745 97.63125) (width 0.2) (layer "F.Cu") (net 1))
 (segment (start 118.745 97.63125) (end 121.44375 100.33) (width 0.2) (layer "F.Cu") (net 1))
 (segment (start 138.181739 98.017989) (end 140.49375 100.33) (width 0.2) (layer "F.Cu") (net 3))
 (segment (start 134.710725 98.017989) (end 138.181739 98.017989) (width 0.2) (layer "F.Cu") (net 3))
 (segment (start 133.82625 86.20125) (end 132.28 86.20125) (width 0.2) (layer "F.Cu") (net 15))
 (segment (start 135.73125 88.10625) (end 133.82625 86.20125) (width 0.2) (layer "F.Cu") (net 15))
 (segment (start 135.73125 90.4875) (end 135.73125 88.10625) (width 0.2) (layer "F.Cu") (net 15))
 (segment (start 102.39375 95.25) (end 102.39375 92.86875) (width 0.2) (layer "F.Cu") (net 15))
 (segment (start 104.775 90.4875) (end 135.73125 90.4875) (width 0.2) (layer "F.Cu") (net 15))
 (segment (start 102.39375 92.86875) (end 104.775 90.4875) (width 0.2) (layer "F.Cu") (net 15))
 (segment (start 136.04875 83.66125) (end 132.28 83.66125) (width 0.2) (layer "F.Cu") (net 16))
 (segment (start 121.44375 95.25) (end 123.825 92.86875) (width 0.2) (layer "F.Cu") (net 16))
 (segment (start 138.1125 85.725) (end 136.04875 83.66125) (width 0.2) (layer "F.Cu") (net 16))
 (segment (start 138.1125 92.86875) (end 138.1125 85.725) (width 0.2) (layer "F.Cu") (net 16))
 (segment (start 123.825 92.86875) (end 138.1125 92.86875) (width 0.2) (layer "F.Cu") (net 16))
 (segment (start 140.49375 83.34375) (end 138.1125 80.9625) (width 0.2) (layer "F.Cu") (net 4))
 (segment (start 137.95375 81.12125) (end 132.28 81.12125) (width 0.2) (layer "F.Cu") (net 4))
 (segment (start 138.1125 80.9625) (end 137.95375 81.12125) (width 0.2) (layer "F.Cu") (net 4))
 (segment (start 140.49375 95.25) (end 140.49375 83.34375) (width 0.2) (layer "F.Cu") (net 4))
 (segment (start 104.408274 100.220476) (end 104.408274 73.81875) (width 0.2) (layer "B.Cu") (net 6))
 (segment (start 104.408274 73.81875) (end 107.265774 70.96125) (width 0.2) (layer "B.Cu") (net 6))
 (segment (start 107.265774 70.96125) (end 116.205 70.96125) (width 0.2) (layer "B.Cu") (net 6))
 (segment (start 97.79 106.83875) (end 104.408274 100.220476) (width 0.2) (layer "B.Cu") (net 6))
 (segment (start 117.1575 106.83875) (end 106.789524 96.470774) (width 0.2) (layer "B.Cu") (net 9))
 (segment (start 106.789524 96.470774) (end 106.789524 76.2) (width 0.2) (layer "B.Cu") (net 9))
 (segment (start 106.789524 76.2) (end 109.488274 73.50125) (width 0.2) (layer "B.Cu") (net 9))
 (segment (start 109.488274 73.50125) (end 116.205 73.50125) (width 0.2) (layer "B.Cu") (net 9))
 (segment (start 109.170774 92.86875) (end 109.170774 78.58125) (width 0.2) (layer "B.Cu") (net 11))
 (segment (start 109.170774 78.58125) (end 111.710774 76.04125) (width 0.2) (layer "B.Cu") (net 11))
 (segment (start 111.710774 76.04125) (end 116.205 76.04125) (width 0.2) (layer "B.Cu") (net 11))
 (segment (start 136.134241 106.894033) (end 122.108958 92.86875) (width 0.2) (layer "B.Cu") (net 11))
 (segment (start 122.108958 92.86875) (end 109.170774 92.86875) (width 0.2) (layer "B.Cu") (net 11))
 (segment (start 153.67 97.63125) (end 156.845 97.63125) (width 0.2) (layer "F.Cu") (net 7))
 (segment (start 156.845 97.63125) (end 159.54375 100.33) (width 0.2) (layer "F.Cu") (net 7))
 (segment (start 154.78125 78.58125) (end 132.28 78.58125) (width 0.2) (layer "F.Cu") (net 8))
 (segment (start 159.54375 95.25) (end 159.54375 83.34375) (width 0.2) (layer "F.Cu") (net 8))
 (segment (start 159.54375 83.34375) (end 154.78125 78.58125) (width 0.2) (layer "F.Cu") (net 8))
 (segment (start 138.707928 90.4875) (end 111.552024 90.4875) (width 0.2) (layer "B.Cu") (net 5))
 (segment (start 111.552024 80.9625) (end 113.933274 78.58125) (width 0.2) (layer "B.Cu") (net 5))
 (segment (start 113.933274 78.58125) (end 116.205 78.58125) (width 0.2) (layer "B.Cu") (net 5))
 (segment (start 111.552024 90.4875) (end 111.552024 80.9625) (width 0.2) (layer "B.Cu") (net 5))
 (segment (start 155.114461 106.894033) (end 138.707928 90.4875) (width 0.2) (layer "B.Cu") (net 5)))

